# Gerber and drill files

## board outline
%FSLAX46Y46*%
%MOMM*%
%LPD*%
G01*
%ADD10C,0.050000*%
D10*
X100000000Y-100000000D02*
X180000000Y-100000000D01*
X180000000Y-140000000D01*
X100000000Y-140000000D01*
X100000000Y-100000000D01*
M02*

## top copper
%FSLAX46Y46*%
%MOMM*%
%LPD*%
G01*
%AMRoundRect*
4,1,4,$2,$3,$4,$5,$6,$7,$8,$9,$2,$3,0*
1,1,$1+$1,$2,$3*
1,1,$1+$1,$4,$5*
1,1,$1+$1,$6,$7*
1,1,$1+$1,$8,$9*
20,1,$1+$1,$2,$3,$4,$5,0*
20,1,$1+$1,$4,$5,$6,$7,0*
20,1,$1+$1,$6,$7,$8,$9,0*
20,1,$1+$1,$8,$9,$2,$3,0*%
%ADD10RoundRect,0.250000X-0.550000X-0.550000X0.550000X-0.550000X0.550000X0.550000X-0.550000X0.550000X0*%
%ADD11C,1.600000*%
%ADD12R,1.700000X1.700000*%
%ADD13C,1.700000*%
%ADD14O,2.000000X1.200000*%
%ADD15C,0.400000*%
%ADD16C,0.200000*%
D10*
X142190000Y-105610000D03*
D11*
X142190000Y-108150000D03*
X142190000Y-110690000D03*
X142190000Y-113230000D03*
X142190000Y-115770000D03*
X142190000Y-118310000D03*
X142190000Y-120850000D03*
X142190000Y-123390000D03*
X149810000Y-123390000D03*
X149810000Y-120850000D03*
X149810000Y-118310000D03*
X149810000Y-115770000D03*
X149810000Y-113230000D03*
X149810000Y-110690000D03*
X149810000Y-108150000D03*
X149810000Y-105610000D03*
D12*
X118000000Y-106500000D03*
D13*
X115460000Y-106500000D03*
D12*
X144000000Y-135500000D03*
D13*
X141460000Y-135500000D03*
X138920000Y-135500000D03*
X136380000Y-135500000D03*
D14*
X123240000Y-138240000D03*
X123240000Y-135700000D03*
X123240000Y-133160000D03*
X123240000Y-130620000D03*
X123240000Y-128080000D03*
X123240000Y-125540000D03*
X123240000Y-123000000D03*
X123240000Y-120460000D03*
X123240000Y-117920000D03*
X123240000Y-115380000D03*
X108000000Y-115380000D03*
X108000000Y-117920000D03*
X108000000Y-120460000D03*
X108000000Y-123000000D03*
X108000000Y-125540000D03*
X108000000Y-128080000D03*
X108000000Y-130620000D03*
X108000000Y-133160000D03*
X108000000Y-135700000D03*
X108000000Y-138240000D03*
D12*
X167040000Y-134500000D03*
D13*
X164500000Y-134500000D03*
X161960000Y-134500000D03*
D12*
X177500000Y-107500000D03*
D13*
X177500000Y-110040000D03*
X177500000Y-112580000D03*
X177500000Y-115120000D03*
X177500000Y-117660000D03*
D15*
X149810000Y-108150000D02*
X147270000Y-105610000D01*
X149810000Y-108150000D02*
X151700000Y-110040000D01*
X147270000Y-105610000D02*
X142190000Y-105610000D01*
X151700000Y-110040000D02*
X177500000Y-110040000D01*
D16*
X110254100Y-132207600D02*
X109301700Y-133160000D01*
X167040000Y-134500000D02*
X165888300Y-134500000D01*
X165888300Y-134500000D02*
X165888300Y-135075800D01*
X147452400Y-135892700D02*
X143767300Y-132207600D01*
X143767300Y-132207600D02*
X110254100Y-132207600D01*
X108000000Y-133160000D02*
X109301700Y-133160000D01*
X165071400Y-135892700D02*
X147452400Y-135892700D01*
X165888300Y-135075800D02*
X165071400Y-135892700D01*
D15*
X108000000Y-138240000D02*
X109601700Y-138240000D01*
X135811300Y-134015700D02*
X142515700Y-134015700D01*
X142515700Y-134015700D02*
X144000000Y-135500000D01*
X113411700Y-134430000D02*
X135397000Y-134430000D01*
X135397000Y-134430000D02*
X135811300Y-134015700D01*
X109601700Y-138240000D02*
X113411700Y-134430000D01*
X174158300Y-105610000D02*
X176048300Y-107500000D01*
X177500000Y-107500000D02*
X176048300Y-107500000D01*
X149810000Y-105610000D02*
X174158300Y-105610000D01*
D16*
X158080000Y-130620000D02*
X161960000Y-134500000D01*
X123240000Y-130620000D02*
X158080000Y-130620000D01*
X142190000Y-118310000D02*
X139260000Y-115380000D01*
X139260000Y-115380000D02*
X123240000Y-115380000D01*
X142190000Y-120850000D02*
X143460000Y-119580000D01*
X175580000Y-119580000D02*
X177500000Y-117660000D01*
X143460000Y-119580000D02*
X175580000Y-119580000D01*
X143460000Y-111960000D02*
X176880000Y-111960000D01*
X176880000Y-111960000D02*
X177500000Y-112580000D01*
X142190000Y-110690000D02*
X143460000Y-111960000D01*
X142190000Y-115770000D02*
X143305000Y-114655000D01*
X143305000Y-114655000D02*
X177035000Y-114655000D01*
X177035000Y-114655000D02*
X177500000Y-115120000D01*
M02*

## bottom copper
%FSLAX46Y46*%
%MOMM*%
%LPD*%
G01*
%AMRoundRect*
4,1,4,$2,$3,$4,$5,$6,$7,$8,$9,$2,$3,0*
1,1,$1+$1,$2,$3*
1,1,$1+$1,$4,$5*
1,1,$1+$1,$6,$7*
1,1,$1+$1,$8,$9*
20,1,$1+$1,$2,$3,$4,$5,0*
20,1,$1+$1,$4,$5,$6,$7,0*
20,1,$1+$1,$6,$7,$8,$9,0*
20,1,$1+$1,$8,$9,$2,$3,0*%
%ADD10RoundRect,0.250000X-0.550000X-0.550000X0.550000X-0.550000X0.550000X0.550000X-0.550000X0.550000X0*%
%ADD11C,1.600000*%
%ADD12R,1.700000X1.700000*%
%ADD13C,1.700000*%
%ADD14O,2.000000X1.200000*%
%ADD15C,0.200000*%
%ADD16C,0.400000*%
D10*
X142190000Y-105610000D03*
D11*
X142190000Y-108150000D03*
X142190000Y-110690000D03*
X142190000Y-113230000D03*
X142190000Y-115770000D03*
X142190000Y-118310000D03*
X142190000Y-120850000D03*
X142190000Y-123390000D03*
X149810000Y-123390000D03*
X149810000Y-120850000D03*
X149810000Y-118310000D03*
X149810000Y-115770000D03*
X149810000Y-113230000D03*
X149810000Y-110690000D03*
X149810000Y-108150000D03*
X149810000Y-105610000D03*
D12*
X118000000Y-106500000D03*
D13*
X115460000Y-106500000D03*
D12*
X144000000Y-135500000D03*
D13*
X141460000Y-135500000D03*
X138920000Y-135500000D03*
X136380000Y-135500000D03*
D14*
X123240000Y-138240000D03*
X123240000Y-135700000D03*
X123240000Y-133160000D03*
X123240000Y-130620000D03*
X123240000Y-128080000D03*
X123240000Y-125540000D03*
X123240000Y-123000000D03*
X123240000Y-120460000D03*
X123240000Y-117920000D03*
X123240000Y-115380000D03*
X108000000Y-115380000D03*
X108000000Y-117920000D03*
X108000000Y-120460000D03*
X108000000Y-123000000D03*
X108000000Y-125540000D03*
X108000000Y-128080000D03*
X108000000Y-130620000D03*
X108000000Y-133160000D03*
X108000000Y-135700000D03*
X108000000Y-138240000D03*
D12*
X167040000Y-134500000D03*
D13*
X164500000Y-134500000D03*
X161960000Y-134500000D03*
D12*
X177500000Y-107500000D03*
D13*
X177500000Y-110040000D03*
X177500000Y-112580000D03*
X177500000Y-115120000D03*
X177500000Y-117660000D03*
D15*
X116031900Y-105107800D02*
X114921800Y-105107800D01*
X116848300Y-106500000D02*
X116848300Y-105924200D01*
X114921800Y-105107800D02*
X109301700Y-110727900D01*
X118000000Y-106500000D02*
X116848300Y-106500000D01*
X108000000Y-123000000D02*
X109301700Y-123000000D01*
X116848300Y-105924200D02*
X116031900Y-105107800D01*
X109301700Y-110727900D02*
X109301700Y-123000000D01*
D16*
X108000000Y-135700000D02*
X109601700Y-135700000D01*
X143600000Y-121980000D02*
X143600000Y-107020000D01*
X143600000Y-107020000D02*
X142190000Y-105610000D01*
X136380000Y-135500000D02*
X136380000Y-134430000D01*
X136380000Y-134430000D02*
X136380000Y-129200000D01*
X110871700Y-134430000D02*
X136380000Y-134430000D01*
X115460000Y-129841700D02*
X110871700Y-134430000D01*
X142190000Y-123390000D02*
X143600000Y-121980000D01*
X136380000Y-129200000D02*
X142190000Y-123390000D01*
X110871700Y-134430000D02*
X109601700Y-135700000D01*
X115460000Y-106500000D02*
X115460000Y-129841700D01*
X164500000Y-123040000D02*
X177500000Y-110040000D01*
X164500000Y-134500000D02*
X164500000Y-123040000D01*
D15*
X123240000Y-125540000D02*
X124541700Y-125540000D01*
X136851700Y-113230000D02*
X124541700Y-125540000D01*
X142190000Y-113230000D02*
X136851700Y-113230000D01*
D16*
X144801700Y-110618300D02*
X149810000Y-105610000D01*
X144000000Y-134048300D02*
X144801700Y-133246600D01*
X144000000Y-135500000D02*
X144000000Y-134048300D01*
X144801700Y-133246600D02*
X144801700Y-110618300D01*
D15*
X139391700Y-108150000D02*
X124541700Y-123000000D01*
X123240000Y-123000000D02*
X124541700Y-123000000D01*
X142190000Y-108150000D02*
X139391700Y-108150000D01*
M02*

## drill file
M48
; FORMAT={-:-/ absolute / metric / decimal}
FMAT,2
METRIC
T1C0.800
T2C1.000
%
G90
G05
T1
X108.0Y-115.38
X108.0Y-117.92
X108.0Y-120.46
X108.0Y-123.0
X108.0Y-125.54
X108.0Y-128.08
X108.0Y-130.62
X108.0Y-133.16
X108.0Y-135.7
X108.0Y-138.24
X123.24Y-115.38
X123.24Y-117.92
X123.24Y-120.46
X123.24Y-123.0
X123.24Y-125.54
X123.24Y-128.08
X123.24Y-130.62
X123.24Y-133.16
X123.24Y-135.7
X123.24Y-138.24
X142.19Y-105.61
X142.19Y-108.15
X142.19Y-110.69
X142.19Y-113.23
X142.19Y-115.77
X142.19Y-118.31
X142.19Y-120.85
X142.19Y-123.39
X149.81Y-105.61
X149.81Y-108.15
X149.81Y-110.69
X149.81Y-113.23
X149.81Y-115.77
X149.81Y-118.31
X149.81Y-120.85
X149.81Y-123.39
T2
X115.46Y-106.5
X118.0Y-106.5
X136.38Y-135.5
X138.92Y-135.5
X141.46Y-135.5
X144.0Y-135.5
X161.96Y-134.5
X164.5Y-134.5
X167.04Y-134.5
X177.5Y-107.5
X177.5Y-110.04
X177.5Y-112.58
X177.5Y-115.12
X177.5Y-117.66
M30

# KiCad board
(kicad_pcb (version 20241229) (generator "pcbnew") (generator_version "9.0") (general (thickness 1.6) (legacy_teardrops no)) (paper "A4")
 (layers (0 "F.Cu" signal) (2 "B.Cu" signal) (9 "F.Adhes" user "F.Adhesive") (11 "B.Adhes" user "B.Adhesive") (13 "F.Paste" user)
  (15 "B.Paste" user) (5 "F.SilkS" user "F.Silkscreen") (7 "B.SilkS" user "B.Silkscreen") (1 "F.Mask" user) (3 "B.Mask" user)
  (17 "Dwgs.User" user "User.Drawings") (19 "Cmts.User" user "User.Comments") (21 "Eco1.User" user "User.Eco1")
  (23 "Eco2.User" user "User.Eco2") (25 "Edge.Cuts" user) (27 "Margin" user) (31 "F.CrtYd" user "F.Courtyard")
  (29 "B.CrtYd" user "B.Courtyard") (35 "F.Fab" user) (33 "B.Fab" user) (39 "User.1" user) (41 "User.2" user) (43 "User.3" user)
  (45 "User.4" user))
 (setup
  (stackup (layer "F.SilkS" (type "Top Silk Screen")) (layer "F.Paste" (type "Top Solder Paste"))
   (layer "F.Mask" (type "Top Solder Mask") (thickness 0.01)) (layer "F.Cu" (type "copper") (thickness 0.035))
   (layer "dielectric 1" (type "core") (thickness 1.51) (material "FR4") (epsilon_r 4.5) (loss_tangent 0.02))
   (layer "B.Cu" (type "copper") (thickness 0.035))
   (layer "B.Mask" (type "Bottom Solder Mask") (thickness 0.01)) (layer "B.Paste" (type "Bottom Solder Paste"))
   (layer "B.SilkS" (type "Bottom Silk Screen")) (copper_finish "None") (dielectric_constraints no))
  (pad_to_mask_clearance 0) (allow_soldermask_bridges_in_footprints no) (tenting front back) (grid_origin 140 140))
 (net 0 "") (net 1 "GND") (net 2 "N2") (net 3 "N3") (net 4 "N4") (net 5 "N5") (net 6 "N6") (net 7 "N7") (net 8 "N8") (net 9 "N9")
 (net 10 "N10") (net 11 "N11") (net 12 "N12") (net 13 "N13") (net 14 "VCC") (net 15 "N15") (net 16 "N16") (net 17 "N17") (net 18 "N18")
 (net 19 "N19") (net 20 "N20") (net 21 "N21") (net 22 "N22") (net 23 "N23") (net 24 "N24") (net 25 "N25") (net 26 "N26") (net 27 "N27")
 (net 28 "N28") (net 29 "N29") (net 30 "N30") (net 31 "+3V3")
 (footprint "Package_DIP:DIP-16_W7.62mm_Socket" (layer "F.Cu") (at 142.19 105.61)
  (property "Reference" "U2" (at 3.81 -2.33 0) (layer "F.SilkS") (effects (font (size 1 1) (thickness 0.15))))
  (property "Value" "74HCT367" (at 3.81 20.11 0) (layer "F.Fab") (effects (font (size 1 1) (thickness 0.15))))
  (pad "1" thru_hole roundrect (at 0 0) (size 1.6 1.6) (drill 0.8) (layers "*.Cu" "*.Mask") (remove_unused_layers no)
   (roundrect_rratio 0.15625) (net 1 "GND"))
  (pad "2" thru_hole circle (at 0 2.54) (size 1.6 1.6) (drill 0.8) (layers "*.Cu" "*.Mask") (remove_unused_layers no) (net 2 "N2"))
  (pad "3" thru_hole circle (at 0 5.08) (size 1.6 1.6) (drill 0.8) (layers "*.Cu" "*.Mask") (remove_unused_layers no) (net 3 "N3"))
  (pad "4" thru_hole circle (at 0 7.62) (size 1.6 1.6) (drill 0.8) (layers "*.Cu" "*.Mask") (remove_unused_layers no) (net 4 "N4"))
  (pad "5" thru_hole circle (at 0 10.16) (size 1.6 1.6) (drill 0.8) (layers "*.Cu" "*.Mask") (remove_unused_layers no) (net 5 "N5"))
  (pad "6" thru_hole circle (at 0 12.7) (size 1.6 1.6) (drill 0.8) (layers "*.Cu" "*.Mask") (remove_unused_layers no) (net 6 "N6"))
  (pad "7" thru_hole circle (at 0 15.24) (size 1.6 1.6) (drill 0.8) (layers "*.Cu" "*.Mask") (remove_unused_layers no) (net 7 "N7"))
  (pad "8" thru_hole circle (at 0 17.78) (size 1.6 1.6) (drill 0.8) (layers "*.Cu" "*.Mask") (remove_unused_layers no) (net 1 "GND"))
  (pad "9" thru_hole circle (at 7.62 17.78) (size 1.6 1.6) (drill 0.8) (layers "*.Cu" "*.Mask") (remove_unused_layers no) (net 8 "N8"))
  (pad "10" thru_hole circle (at 7.62 15.24) (size 1.6 1.6) (drill 0.8) (layers "*.Cu" "*.Mask") (remove_unused_layers no) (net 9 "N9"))
  (pad "11" thru_hole circle (at 7.62 12.7) (size 1.6 1.6) (drill 0.8) (layers "*.Cu" "*.Mask") (remove_unused_layers no) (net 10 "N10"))
  (pad "12" thru_hole circle (at 7.62 10.16) (size 1.6 1.6) (drill 0.8) (layers "*.Cu" "*.Mask") (remove_unused_layers no) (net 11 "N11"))
  (pad "13" thru_hole circle (at 7.62 7.62) (size 1.6 1.6) (drill 0.8) (layers "*.Cu" "*.Mask") (remove_unused_layers no) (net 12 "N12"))
  (pad "14" thru_hole circle (at 7.62 5.08) (size 1.6 1.6) (drill 0.8) (layers "*.Cu" "*.Mask") (remove_unused_layers no) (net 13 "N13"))
  (pad "15" thru_hole circle (at 7.62 2.54) (size 1.6 1.6) (drill 0.8) (layers "*.Cu" "*.Mask") (remove_unused_layers no) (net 1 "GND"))
  (pad "16" thru_hole circle (at 7.62 0) (size 1.6 1.6) (drill 0.8) (layers "*.Cu" "*.Mask") (remove_unused_layers no) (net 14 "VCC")))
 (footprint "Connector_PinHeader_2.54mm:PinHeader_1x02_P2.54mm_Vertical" (layer "F.Cu") (at 118 106.5 -90)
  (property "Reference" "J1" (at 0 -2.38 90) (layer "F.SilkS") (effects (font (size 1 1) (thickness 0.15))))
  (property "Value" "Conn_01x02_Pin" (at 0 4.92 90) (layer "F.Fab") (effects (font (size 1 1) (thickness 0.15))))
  (pad "1" thru_hole rect (at 0 0 270) (size 1.7 1.7) (drill 1) (layers "*.Cu" "*.Mask") (remove_unused_layers no) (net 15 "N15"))
  (pad "2" thru_hole circle (at 0 2.54 270) (size 1.7 1.7) (drill 1) (layers "*.Cu" "*.Mask") (remove_unused_layers no) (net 1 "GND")))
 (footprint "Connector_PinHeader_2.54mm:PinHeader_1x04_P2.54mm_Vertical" (layer "F.Cu") (at 144 135.5 -90)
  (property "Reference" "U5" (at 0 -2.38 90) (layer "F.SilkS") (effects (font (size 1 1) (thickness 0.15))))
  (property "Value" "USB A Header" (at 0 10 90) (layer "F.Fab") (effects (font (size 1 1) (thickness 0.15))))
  (pad "1" thru_hole rect (at 0 0 270) (size 1.7 1.7) (drill 1) (layers "*.Cu" "*.Mask") (remove_unused_layers no) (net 14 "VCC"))
  (pad "2" thru_hole circle (at 0 2.54 270) (size 1.7 1.7) (drill 1) (layers "*.Cu" "*.Mask") (remove_unused_layers no) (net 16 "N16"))
  (pad "3" thru_hole circle (at 0 5.08 270) (size 1.7 1.7) (drill 1) (layers "*.Cu" "*.Mask") (remove_unused_layers no) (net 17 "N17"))
  (pad "4" thru_hole circle (at 0 7.62 270) (size 1.7 1.7) (drill 1) (layers "*.Cu" "*.Mask") (remove_unused_layers no) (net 1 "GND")))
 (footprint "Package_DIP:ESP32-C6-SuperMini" (layer "F.Cu") (at 115.62 126.81)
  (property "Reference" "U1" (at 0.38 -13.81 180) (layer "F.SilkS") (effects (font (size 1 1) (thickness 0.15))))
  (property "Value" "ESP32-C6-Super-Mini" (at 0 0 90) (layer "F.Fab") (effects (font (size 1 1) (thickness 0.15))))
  (pad "1" thru_hole oval (at 7.62 11.43 90) (size 1.2 2) (drill 0.8) (layers "*.Cu" "*.Mask") (remove_unused_layers no) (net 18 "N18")
   (thermal_bridge_angle 45))
  (pad "2" thru_hole oval (at 7.62 8.89 90) (size 1.2 2) (drill 0.8) (layers "*.Cu" "*.Mask") (remove_unused_layers no) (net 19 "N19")
   (thermal_bridge_angle 45))
  (pad "3" thru_hole oval (at 7.62 6.35 90) (size 1.2 2) (drill 0.8) (layers "*.Cu" "*.Mask") (remove_unused_layers no) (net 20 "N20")
   (thermal_bridge_angle 45))
  (pad "4" thru_hole oval (at 7.62 3.81 90) (size 1.2 2) (drill 0.8) (layers "*.Cu" "*.Mask") (remove_unused_layers no) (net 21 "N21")
   (thermal_bridge_angle 45))
  (pad "5" thru_hole oval (at 7.62 1.27 90) (size 1.2 2) (drill 0.8) (layers "*.Cu" "*.Mask") (remove_unused_layers no) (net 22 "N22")
   (thermal_bridge_angle 45))
  (pad "6" thru_hole oval (at 7.62 -1.27 90) (size 1.2 2) (drill 0.8) (layers "*.Cu" "*.Mask") (remove_unused_layers no) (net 4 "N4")
   (thermal_bridge_angle 45))
  (pad "7" thru_hole oval (at 7.62 -3.81 90) (size 1.2 2) (drill 0.8) (layers "*.Cu" "*.Mask") (remove_unused_layers no) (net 2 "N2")
   (thermal_bridge_angle 45))
  (pad "8" thru_hole oval (at 7.62 -6.35 90) (size 1.2 2) (drill 0.8) (layers "*.Cu" "*.Mask") (remove_unused_layers no) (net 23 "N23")
   (thermal_bridge_angle 45))
  (pad "9" thru_hole oval (at 7.62 -8.89 90) (size 1.2 2) (drill 0.8) (layers "*.Cu" "*.Mask") (remove_unused_layers no) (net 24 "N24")
   (thermal_bridge_angle 45))
  (pad "10" thru_hole oval (at 7.62 -11.43 90) (size 1.2 2) (drill 0.8) (layers "*.Cu" "*.Mask") (remove_unused_layers no) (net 6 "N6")
   (thermal_bridge_angle 45))
  (pad "11" thru_hole oval (at -7.62 -11.43 90) (size 1.2 2) (drill 0.8) (layers "*.Cu" "*.Mask") (remove_unused_layers no) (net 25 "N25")
   (thermal_bridge_angle 45))
  (pad "12" thru_hole oval (at -7.62 -8.89 90) (size 1.2 2) (drill 0.8) (layers "*.Cu" "*.Mask") (remove_unused_layers no) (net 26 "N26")
   (thermal_bridge_angle 45))
  (pad "13" thru_hole oval (at -7.62 -6.35 90) (size 1.2 2) (drill 0.8) (layers "*.Cu" "*.Mask") (remove_unused_layers no) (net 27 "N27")
   (thermal_bridge_angle 45))
  (pad "14" thru_hole oval (at -7.62 -3.81 90) (size 1.2 2) (drill 0.8) (layers "*.Cu" "*.Mask") (remove_unused_layers no) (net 15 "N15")
   (thermal_bridge_angle 45))
  (pad "15" thru_hole oval (at -7.62 -1.27 90) (size 1.2 2) (drill 0.8) (layers "*.Cu" "*.Mask") (remove_unused_layers no) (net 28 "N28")
   (thermal_bridge_angle 45))
  (pad "16" thru_hole oval (at -7.62 1.27 90) (size 1.2 2) (drill 0.8) (layers "*.Cu" "*.Mask") (remove_unused_layers no) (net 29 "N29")
   (thermal_bridge_angle 45))
  (pad "17" thru_hole oval (at -7.62 3.81 90) (size 1.2 2) (drill 0.8) (layers "*.Cu" "*.Mask") (remove_unused_layers no) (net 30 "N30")
   (thermal_bridge_angle 45))
  (pad "18" thru_hole oval (at -7.62 6.35 90) (size 1.2 2) (drill 0.8) (layers "*.Cu" "*.Mask") (remove_unused_layers no) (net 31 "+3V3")
   (thermal_bridge_angle 45))
  (pad "19" thru_hole oval (at -7.62 8.89 90) (size 1.2 2) (drill 0.8) (layers "*.Cu" "*.Mask") (remove_unused_layers no) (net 1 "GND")
   (thermal_bridge_angle 45))
  (pad "20" thru_hole oval (at -7.62 11.43 90) (size 1.2 2) (drill 0.8) (layers "*.Cu" "*.Mask") (remove_unused_layers no) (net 14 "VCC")
   (thermal_bridge_angle 45)))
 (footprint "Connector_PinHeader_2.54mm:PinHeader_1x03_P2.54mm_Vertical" (layer "B.Cu") (at 167.04 134.5 90)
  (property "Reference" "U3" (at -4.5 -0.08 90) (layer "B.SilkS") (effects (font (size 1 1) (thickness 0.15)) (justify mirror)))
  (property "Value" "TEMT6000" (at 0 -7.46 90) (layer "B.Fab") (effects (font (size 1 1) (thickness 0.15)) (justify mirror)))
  (pad "1" thru_hole rect (at 0 0 90) (size 1.7 1.7) (drill 1) (layers "*.Cu" "*.Mask") (remove_unused_layers no) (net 31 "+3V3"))
  (pad "2" thru_hole circle (at 0 -2.54 90) (size 1.7 1.7) (drill 1) (layers "*.Cu" "*.Mask") (remove_unused_layers no) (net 1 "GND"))
  (pad "3" thru_hole circle (at 0 -5.08 90) (size 1.7 1.7) (drill 1) (layers "*.Cu" "*.Mask") (remove_unused_layers no) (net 21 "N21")))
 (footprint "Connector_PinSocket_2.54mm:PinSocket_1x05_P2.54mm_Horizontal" (layer "B.Cu") (at 168.5 107.5 180)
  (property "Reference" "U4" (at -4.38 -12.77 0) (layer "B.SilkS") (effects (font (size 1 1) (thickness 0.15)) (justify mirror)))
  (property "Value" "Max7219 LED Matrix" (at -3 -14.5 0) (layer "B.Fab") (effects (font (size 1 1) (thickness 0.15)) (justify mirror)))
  (pad "1" thru_hole rect (at -9 0 180) (size 1.7 1.7) (drill 1) (layers "*.Cu" "*.Mask") (remove_unused_layers no) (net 14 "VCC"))
  (pad "2" thru_hole circle (at -9 -2.54 180) (size 1.7 1.7) (drill 1) (layers "*.Cu" "*.Mask") (remove_unused_layers no) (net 1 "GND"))
  (pad "3" thru_hole circle (at -9 -5.08 180) (size 1.7 1.7) (drill 1) (layers "*.Cu" "*.Mask") (remove_unused_layers no) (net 3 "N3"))
  (pad "4" thru_hole circle (at -9 -7.62 180) (size 1.7 1.7) (drill 1) (layers "*.Cu" "*.Mask") (remove_unused_layers no) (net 5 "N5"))
  (pad "5" thru_hole circle (at -9 -10.16 180) (size 1.7 1.7) (drill 1) (layers "*.Cu" "*.Mask") (remove_unused_layers no) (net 7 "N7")))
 (gr_rect (start 100 100) (end 180 140) (stroke (width 0.05) (type solid)) (fill no) (layer "Edge.Cuts"))
 (segment (start 116.0319 105.1078) (end 114.9218 105.1078) (width 0.2) (layer "B.Cu") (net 15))
 (segment (start 116.8483 106.5) (end 116.8483 105.9242) (width 0.2) (layer "B.Cu") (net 15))
 (segment (start 114.9218 105.1078) (end 109.3017 110.7279) (width 0.2) (layer "B.Cu") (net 15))
 (segment (start 118 106.5) (end 116.8483 106.5) (width 0.2) (layer "B.Cu") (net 15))
 (segment (start 108 123) (end 109.3017 123) (width 0.2) (layer "B.Cu") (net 15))
 (segment (start 116.8483 105.9242) (end 116.0319 105.1078) (width 0.2) (layer "B.Cu") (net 15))
 (segment (start 109.3017 110.7279) (end 109.3017 123) (width 0.2) (layer "B.Cu") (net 15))
 (segment (start 149.81 108.15) (end 147.27 105.61) (width 0.4) (layer "F.Cu") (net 1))
 (segment (start 149.81 108.15) (end 151.7 110.04) (width 0.4) (layer "F.Cu") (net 1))
 (segment (start 147.27 105.61) (end 142.19 105.61) (width 0.4) (layer "F.Cu") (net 1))
 (segment (start 151.7 110.04) (end 177.5 110.04) (width 0.4) (layer "F.Cu") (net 1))
 (segment (start 108 135.7) (end 109.6017 135.7) (width 0.4) (layer "B.Cu") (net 1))
 (segment (start 143.6 121.98) (end 143.6 107.02) (width 0.4) (layer "B.Cu") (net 1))
 (segment (start 143.6 107.02) (end 142.19 105.61) (width 0.4) (layer "B.Cu") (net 1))
 (segment (start 136.38 135.5) (end 136.38 134.43) (width 0.4) (layer "B.Cu") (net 1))
 (segment (start 136.38 134.43) (end 136.38 129.2) (width 0.4) (layer "B.Cu") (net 1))
 (segment (start 110.8717 134.43) (end 136.38 134.43) (width 0.4) (layer "B.Cu") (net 1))
 (segment (start 115.46 129.8417) (end 110.8717 134.43) (width 0.4) (layer "B.Cu") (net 1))
 (segment (start 142.19 123.39) (end 143.6 121.98) (width 0.4) (layer "B.Cu") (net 1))
 (segment (start 136.38 129.2) (end 142.19 123.39) (width 0.4) (layer "B.Cu") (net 1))
 (segment (start 110.8717 134.43) (end 109.6017 135.7) (width 0.4) (layer "B.Cu") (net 1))
 (segment (start 115.46 106.5) (end 115.46 129.8417) (width 0.4) (layer "B.Cu") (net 1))
 (segment (start 164.5 123.04) (end 177.5 110.04) (width 0.4) (layer "B.Cu") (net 1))
 (segment (start 164.5 134.5) (end 164.5 123.04) (width 0.4) (layer "B.Cu") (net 1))
 (segment (start 110.2541 132.2076) (end 109.3017 133.16) (width 0.2) (layer "F.Cu") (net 31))
 (segment (start 167.04 134.5) (end 165.8883 134.5) (width 0.2) (layer "F.Cu") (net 31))
 (segment (start 165.8883 134.5) (end 165.8883 135.0758) (width 0.2) (layer "F.Cu") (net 31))
 (segment (start 147.4524 135.8927) (end 143.7673 132.2076) (width 0.2) (layer "F.Cu") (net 31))
 (segment (start 143.7673 132.2076) (end 110.2541 132.2076) (width 0.2) (layer "F.Cu") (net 31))
 (segment (start 108 133.16) (end 109.3017 133.16) (width 0.2) (layer "F.Cu") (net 31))
 (segment (start 165.0714 135.8927) (end 147.4524 135.8927) (width 0.2) (layer "F.Cu") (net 31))
 (segment (start 165.8883 135.0758) (end 165.0714 135.8927) (width 0.2) (layer "F.Cu") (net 31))
 (segment (start 123.24 125.54) (end 124.5417 125.54) (width 0.2) (layer "B.Cu") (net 4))
 (segment (start 136.8517 113.23) (end 124.5417 125.54) (width 0.2) (layer "B.Cu") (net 4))
 (segment (start 142.19 113.23) (end 136.8517 113.23) (width 0.2) (layer "B.Cu") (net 4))
 (segment (start 108 138.24) (end 109.6017 138.24) (width 0.4) (layer "F.Cu") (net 14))
 (segment (start 135.8113 134.0157) (end 142.5157 134.0157) (width 0.4) (layer "F.Cu") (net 14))
 (segment (start 142.5157 134.0157) (end 144 135.5) (width 0.4) (layer "F.Cu") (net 14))
 (segment (start 113.4117 134.43) (end 135.397 134.43) (width 0.4) (layer "F.Cu") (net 14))
 (segment (start 135.397 134.43) (end 135.8113 134.0157) (width 0.4) (layer "F.Cu") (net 14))
 (segment (start 109.6017 138.24) (end 113.4117 134.43) (width 0.4) (layer "F.Cu") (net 14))
 (segment (start 174.1583 105.61) (end 176.0483 107.5) (width 0.4) (layer "F.Cu") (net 14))
 (segment (start 177.5 107.5) (end 176.0483 107.5) (width 0.4) (layer "F.Cu") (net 14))
 (segment (start 149.81 105.61) (end 174.1583 105.61) (width 0.4) (layer "F.Cu") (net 14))
 (segment (start 144.8017 110.6183) (end 149.81 105.61) (width 0.4) (layer "B.Cu") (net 14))
 (segment (start 144 134.0483) (end 144.8017 133.2466) (width 0.4) (layer "B.Cu") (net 14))
 (segment (start 144 135.5) (end 144 134.0483) (width 0.4) (layer "B.Cu") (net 14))
 (segment (start 144.8017 133.2466) (end 144.8017 110.6183) (width 0.4) (layer "B.Cu") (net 14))
 (segment (start 139.3917 108.15) (end 124.5417 123) (width 0.2) (layer "B.Cu") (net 2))
 (segment (start 123.24 123) (end 124.5417 123) (width 0.2) (layer "B.Cu") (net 2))
 (segment (start 142.19 108.15) (end 139.3917 108.15) (width 0.2) (layer "B.Cu") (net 2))
 (segment (start 158.08 130.62) (end 161.96 134.5) (width 0.2) (layer "F.Cu") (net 21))
 (segment (start 123.24 130.62) (end 158.08 130.62) (width 0.2) (layer "F.Cu") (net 21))
 (segment (start 142.19 118.31) (end 139.26 115.38) (width 0.2) (layer "F.Cu") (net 6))
 (segment (start 139.26 115.38) (end 123.24 115.38) (width 0.2) (layer "F.Cu") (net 6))
 (segment (start 142.19 120.85) (end 143.46 119.58) (width 0.2) (layer "F.Cu") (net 7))
 (segment (start 175.58 119.58) (end 177.5 117.66) (width 0.2) (layer "F.Cu") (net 7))
 (segment (start 143.46 119.58) (end 175.58 119.58) (width 0.2) (layer "F.Cu") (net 7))
 (segment (start 143.46 111.96) (end 176.88 111.96) (width 0.2) (layer "F.Cu") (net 3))
 (segment (start 176.88 111.96) (end 177.5 112.58) (width 0.2) (layer "F.Cu") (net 3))
 (segment (start 142.19 110.69) (end 143.46 111.96) (width 0.2) (layer "F.Cu") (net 3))
 (segment (start 142.19 115.77) (end 143.305 114.655) (width 0.2) (layer "F.Cu") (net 5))
 (segment (start 143.305 114.655) (end 177.035 114.655) (width 0.2) (layer "F.Cu") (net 5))
 (segment (start 177.035 114.655) (end 177.5 115.12) (width 0.2) (layer "F.Cu") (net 5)))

